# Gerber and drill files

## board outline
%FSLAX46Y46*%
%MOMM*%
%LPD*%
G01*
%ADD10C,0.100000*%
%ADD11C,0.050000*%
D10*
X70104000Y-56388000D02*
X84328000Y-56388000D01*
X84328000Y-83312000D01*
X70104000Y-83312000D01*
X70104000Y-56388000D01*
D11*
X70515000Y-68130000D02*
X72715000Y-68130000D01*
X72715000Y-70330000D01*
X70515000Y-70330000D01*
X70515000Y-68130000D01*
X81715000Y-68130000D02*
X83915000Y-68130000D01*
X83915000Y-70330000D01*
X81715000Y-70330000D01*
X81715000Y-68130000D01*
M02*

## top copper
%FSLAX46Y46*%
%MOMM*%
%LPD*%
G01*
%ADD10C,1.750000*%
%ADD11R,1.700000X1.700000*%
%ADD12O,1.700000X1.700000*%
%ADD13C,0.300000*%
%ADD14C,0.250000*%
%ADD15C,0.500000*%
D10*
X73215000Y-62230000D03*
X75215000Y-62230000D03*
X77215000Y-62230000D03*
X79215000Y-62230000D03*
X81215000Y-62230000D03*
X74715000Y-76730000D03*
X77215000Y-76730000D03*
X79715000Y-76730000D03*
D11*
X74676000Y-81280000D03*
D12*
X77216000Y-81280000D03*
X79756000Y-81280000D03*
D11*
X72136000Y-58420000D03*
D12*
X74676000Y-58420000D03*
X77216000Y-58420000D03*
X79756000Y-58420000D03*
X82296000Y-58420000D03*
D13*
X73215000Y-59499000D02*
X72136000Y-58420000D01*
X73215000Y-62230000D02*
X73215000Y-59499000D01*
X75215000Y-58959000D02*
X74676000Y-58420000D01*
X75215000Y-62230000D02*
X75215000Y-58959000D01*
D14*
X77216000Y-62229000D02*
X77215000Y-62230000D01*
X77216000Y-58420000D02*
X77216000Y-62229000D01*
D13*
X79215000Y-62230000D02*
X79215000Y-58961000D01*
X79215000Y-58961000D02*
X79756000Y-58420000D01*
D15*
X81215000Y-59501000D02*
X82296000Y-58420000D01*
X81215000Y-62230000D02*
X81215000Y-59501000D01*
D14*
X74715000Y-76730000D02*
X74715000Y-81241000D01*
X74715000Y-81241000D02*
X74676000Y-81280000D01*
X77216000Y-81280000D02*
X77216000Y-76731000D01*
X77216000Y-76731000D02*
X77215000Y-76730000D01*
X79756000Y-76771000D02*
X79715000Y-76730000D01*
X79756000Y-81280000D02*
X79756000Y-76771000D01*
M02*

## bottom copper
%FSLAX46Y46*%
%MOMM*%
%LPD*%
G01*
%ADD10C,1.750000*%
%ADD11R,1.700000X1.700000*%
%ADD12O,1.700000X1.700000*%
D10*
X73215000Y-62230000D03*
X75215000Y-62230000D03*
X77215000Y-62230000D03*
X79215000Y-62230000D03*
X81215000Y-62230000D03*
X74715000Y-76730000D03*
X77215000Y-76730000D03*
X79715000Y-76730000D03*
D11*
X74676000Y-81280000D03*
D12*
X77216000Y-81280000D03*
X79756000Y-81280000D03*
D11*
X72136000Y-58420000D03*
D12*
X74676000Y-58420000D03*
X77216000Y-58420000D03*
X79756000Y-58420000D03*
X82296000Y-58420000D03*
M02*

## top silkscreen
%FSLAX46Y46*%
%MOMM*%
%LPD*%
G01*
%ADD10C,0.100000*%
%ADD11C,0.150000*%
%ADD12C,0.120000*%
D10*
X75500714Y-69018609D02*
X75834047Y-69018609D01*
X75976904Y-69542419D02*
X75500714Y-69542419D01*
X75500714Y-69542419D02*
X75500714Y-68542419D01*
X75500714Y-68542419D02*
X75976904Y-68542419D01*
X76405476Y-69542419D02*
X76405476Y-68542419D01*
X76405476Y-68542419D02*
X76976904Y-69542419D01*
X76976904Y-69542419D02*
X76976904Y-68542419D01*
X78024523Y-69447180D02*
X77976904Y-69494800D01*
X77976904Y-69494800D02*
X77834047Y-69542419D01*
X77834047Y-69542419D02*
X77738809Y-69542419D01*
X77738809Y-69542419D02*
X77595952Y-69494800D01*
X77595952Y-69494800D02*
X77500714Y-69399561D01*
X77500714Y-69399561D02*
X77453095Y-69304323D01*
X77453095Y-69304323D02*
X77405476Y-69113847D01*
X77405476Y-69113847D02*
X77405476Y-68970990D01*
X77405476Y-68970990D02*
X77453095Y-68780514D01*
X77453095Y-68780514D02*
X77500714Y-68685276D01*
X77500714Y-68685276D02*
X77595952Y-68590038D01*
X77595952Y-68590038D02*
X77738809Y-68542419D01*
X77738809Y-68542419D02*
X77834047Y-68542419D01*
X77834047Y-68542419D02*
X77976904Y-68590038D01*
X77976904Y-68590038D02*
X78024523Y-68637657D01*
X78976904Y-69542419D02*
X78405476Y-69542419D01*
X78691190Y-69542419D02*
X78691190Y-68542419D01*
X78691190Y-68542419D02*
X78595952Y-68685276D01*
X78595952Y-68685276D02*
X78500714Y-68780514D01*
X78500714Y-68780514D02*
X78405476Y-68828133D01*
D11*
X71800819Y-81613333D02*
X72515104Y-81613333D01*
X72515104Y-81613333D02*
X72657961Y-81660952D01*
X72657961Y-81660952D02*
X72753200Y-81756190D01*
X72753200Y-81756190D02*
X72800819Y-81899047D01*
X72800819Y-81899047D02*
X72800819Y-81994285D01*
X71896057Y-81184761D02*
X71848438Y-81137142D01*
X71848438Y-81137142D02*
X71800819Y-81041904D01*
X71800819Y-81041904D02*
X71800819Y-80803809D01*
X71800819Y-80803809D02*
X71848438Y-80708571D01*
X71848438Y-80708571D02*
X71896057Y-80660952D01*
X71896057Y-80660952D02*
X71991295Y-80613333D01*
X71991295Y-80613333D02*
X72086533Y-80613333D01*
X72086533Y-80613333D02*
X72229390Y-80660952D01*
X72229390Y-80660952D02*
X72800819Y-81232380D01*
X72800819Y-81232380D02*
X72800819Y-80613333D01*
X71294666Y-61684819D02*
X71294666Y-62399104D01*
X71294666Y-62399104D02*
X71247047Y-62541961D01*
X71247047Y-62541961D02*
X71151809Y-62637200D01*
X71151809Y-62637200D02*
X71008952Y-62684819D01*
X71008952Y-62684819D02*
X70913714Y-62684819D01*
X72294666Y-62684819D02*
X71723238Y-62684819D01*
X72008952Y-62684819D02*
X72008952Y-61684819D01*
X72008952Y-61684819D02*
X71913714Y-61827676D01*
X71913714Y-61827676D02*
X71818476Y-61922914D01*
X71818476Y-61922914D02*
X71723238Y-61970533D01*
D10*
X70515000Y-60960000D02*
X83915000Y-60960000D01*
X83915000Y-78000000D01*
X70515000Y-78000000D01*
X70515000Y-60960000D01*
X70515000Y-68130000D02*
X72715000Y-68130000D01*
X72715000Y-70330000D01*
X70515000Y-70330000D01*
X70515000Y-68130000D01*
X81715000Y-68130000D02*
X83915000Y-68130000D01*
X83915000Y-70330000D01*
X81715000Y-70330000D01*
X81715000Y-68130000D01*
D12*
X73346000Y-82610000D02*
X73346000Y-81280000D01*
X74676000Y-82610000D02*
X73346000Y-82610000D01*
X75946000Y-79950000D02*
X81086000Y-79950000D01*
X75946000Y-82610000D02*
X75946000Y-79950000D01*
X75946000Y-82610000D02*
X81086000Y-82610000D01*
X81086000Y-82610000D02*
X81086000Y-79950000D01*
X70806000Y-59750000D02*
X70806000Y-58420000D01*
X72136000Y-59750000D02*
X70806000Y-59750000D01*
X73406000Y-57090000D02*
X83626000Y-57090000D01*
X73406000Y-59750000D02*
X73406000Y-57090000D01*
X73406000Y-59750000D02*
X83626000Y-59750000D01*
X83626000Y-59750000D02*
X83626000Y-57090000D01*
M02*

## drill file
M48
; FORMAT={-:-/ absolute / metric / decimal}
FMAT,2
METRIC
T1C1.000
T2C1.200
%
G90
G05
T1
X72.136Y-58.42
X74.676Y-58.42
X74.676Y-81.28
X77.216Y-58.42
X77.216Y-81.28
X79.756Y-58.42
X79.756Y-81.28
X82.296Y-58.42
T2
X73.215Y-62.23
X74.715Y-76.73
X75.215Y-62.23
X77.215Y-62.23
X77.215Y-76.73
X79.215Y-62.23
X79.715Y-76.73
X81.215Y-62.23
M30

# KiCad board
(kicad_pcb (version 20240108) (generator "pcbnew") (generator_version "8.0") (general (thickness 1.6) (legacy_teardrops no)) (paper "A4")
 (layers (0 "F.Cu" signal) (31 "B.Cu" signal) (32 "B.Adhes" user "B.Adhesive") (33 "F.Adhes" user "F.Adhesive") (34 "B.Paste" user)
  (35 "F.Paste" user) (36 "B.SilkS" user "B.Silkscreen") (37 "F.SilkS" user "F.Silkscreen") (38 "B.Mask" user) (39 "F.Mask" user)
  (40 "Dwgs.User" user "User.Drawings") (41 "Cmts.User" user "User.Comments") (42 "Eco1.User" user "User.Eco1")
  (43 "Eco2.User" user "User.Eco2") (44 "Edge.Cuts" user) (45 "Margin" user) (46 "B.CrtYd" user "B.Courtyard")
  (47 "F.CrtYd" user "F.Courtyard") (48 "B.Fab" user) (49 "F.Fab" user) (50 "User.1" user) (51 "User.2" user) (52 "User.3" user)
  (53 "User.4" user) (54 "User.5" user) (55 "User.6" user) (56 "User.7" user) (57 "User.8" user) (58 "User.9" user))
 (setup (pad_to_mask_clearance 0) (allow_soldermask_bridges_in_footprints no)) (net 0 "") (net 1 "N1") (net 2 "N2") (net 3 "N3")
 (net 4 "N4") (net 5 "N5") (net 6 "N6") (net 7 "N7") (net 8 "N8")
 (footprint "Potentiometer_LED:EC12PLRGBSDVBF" (layer "F.Cu") (at 77.215 69.23)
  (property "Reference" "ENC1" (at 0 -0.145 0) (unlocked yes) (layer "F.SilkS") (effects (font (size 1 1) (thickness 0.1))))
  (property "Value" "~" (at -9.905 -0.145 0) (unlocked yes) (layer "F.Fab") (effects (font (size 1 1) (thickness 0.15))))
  (fp_rect (start -6.7 -8.27) (end 6.7 8.77) (stroke (width 0.1) (type default)) (fill none) (layer "F.SilkS"))
  (fp_rect (start -4.5 -1.1) (end -6.7 1.1) (stroke (width 0.1) (type default)) (fill none) (layer "F.SilkS"))
  (fp_rect (start 4.5 -1.1) (end 6.7 1.1) (stroke (width 0.1) (type default)) (fill none) (layer "F.SilkS"))
  (fp_rect (start -6.7 -1.1) (end -4.5 1.1) (stroke (width 0.05) (type default)) (fill none) (layer "Edge.Cuts"))
  (fp_rect (start 4.5 -1.1) (end 6.7 1.1) (stroke (width 0.05) (type default)) (fill none) (layer "Edge.Cuts"))
  (pad "1" thru_hole circle (at -4 -7) (size 1.75 1.75) (drill 1.2) (layers "*.Cu" "*.Mask") (remove_unused_layers no) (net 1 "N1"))
  (pad "2" thru_hole circle (at -2 -7) (size 1.75 1.75) (drill 1.2) (layers "*.Cu" "*.Mask") (remove_unused_layers no) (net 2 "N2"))
  (pad "3" thru_hole circle (at 0 -7) (size 1.75 1.75) (drill 1.2) (layers "*.Cu" "*.Mask") (remove_unused_layers no) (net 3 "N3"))
  (pad "4" thru_hole circle (at 2 -7) (size 1.75 1.75) (drill 1.2) (layers "*.Cu" "*.Mask") (remove_unused_layers no) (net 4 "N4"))
  (pad "5" thru_hole circle (at 4 -7) (size 1.75 1.75) (drill 1.2) (layers "*.Cu" "*.Mask") (remove_unused_layers no) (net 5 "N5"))
  (pad "6" thru_hole circle (at -2.5 7.5) (size 1.75 1.75) (drill 1.2) (layers "*.Cu" "*.Mask") (remove_unused_layers no) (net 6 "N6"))
  (pad "7" thru_hole circle (at 0 7.5) (size 1.75 1.75) (drill 1.2) (layers "*.Cu" "*.Mask") (remove_unused_layers no) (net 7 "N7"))
  (pad "8" thru_hole circle (at 2.5 7.5) (size 1.75 1.75) (drill 1.2) (layers "*.Cu" "*.Mask") (remove_unused_layers no) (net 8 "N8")))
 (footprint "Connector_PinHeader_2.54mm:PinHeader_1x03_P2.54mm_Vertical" (layer "F.Cu") (at 74.676 81.28 90)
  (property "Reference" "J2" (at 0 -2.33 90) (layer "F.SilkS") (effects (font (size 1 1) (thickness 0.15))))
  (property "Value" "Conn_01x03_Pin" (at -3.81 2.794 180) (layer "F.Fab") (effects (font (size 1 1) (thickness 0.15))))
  (fp_line (start -1.33 -1.33) (end 0 -1.33) (stroke (width 0.12) (type solid)) (layer "F.SilkS"))
  (fp_line (start -1.33 0) (end -1.33 -1.33) (stroke (width 0.12) (type solid)) (layer "F.SilkS"))
  (fp_line (start 1.33 1.27) (end 1.33 6.41) (stroke (width 0.12) (type solid)) (layer "F.SilkS"))
  (fp_line (start -1.33 1.27) (end 1.33 1.27) (stroke (width 0.12) (type solid)) (layer "F.SilkS"))
  (fp_line (start -1.33 1.27) (end -1.33 6.41) (stroke (width 0.12) (type solid)) (layer "F.SilkS"))
  (fp_line (start -1.33 6.41) (end 1.33 6.41) (stroke (width 0.12) (type solid)) (layer "F.SilkS"))
  (pad "1" thru_hole rect (at 0 0 90) (size 1.7 1.7) (drill 1) (layers "*.Cu" "*.Mask") (remove_unused_layers no) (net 6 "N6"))
  (pad "2" thru_hole oval (at 0 2.54 90) (size 1.7 1.7) (drill 1) (layers "*.Cu" "*.Mask") (remove_unused_layers no) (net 7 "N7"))
  (pad "3" thru_hole oval (at 0 5.08 90) (size 1.7 1.7) (drill 1) (layers "*.Cu" "*.Mask") (remove_unused_layers no) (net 8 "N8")))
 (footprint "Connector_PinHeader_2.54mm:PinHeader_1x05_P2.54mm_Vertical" (layer "F.Cu") (at 72.136 58.42 90)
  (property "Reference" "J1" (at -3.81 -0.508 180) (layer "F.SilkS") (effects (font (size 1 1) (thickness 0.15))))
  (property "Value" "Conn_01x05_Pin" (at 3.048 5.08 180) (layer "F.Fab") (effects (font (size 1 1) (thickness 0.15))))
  (fp_line (start -1.33 -1.33) (end 0 -1.33) (stroke (width 0.12) (type solid)) (layer "F.SilkS"))
  (fp_line (start -1.33 0) (end -1.33 -1.33) (stroke (width 0.12) (type solid)) (layer "F.SilkS"))
  (fp_line (start 1.33 1.27) (end 1.33 11.49) (stroke (width 0.12) (type solid)) (layer "F.SilkS"))
  (fp_line (start -1.33 1.27) (end 1.33 1.27) (stroke (width 0.12) (type solid)) (layer "F.SilkS"))
  (fp_line (start -1.33 1.27) (end -1.33 11.49) (stroke (width 0.12) (type solid)) (layer "F.SilkS"))
  (fp_line (start -1.33 11.49) (end 1.33 11.49) (stroke (width 0.12) (type solid)) (layer "F.SilkS"))
  (pad "1" thru_hole rect (at 0 0 90) (size 1.7 1.7) (drill 1) (layers "*.Cu" "*.Mask") (remove_unused_layers no) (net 1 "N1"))
  (pad "2" thru_hole oval (at 0 2.54 90) (size 1.7 1.7) (drill 1) (layers "*.Cu" "*.Mask") (remove_unused_layers no) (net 2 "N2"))
  (pad "3" thru_hole oval (at 0 5.08 90) (size 1.7 1.7) (drill 1) (layers "*.Cu" "*.Mask") (remove_unused_layers no) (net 3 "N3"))
  (pad "4" thru_hole oval (at 0 7.62 90) (size 1.7 1.7) (drill 1) (layers "*.Cu" "*.Mask") (remove_unused_layers no) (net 4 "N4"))
  (pad "5" thru_hole oval (at 0 10.16 90) (size 1.7 1.7) (drill 1) (layers "*.Cu" "*.Mask") (remove_unused_layers no) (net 5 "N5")))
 (gr_rect (start 70.104 56.388) (end 84.328 83.312) (stroke (width 0.1) (type default)) (fill none) (layer "Edge.Cuts"))
 (segment (start 73.215 59.499) (end 72.136 58.42) (width 0.3) (layer "F.Cu") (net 1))
 (segment (start 73.215 62.23) (end 73.215 59.499) (width 0.3) (layer "F.Cu") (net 1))
 (segment (start 75.215 58.959) (end 74.676 58.42) (width 0.3) (layer "F.Cu") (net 2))
 (segment (start 75.215 62.23) (end 75.215 58.959) (width 0.3) (layer "F.Cu") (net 2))
 (segment (start 77.216 62.229) (end 77.215 62.23) (width 0.25) (layer "F.Cu") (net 3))
 (segment (start 77.216 58.42) (end 77.216 62.229) (width 0.25) (layer "F.Cu") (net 3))
 (segment (start 79.215 62.23) (end 79.215 58.961) (width 0.3) (layer "F.Cu") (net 4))
 (segment (start 79.215 58.961) (end 79.756 58.42) (width 0.3) (layer "F.Cu") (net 4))
 (segment (start 81.215 59.501) (end 82.296 58.42) (width 0.5) (layer "F.Cu") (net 5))
 (segment (start 81.215 62.23) (end 81.215 59.501) (width 0.5) (layer "F.Cu") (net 5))
 (segment (start 74.715 76.73) (end 74.715 81.241) (width 0.25) (layer "F.Cu") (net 6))
 (segment (start 74.715 81.241) (end 74.676 81.28) (width 0.25) (layer "F.Cu") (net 6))
 (segment (start 77.216 81.28) (end 77.216 76.731) (width 0.25) (layer "F.Cu") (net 7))
 (segment (start 77.216 76.731) (end 77.215 76.73) (width 0.25) (layer "F.Cu") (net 7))
 (segment (start 79.756 76.771) (end 79.715 76.73) (width 0.25) (layer "F.Cu") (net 8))
 (segment (start 79.756 81.28) (end 79.756 76.771) (width 0.25) (layer "F.Cu") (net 8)))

